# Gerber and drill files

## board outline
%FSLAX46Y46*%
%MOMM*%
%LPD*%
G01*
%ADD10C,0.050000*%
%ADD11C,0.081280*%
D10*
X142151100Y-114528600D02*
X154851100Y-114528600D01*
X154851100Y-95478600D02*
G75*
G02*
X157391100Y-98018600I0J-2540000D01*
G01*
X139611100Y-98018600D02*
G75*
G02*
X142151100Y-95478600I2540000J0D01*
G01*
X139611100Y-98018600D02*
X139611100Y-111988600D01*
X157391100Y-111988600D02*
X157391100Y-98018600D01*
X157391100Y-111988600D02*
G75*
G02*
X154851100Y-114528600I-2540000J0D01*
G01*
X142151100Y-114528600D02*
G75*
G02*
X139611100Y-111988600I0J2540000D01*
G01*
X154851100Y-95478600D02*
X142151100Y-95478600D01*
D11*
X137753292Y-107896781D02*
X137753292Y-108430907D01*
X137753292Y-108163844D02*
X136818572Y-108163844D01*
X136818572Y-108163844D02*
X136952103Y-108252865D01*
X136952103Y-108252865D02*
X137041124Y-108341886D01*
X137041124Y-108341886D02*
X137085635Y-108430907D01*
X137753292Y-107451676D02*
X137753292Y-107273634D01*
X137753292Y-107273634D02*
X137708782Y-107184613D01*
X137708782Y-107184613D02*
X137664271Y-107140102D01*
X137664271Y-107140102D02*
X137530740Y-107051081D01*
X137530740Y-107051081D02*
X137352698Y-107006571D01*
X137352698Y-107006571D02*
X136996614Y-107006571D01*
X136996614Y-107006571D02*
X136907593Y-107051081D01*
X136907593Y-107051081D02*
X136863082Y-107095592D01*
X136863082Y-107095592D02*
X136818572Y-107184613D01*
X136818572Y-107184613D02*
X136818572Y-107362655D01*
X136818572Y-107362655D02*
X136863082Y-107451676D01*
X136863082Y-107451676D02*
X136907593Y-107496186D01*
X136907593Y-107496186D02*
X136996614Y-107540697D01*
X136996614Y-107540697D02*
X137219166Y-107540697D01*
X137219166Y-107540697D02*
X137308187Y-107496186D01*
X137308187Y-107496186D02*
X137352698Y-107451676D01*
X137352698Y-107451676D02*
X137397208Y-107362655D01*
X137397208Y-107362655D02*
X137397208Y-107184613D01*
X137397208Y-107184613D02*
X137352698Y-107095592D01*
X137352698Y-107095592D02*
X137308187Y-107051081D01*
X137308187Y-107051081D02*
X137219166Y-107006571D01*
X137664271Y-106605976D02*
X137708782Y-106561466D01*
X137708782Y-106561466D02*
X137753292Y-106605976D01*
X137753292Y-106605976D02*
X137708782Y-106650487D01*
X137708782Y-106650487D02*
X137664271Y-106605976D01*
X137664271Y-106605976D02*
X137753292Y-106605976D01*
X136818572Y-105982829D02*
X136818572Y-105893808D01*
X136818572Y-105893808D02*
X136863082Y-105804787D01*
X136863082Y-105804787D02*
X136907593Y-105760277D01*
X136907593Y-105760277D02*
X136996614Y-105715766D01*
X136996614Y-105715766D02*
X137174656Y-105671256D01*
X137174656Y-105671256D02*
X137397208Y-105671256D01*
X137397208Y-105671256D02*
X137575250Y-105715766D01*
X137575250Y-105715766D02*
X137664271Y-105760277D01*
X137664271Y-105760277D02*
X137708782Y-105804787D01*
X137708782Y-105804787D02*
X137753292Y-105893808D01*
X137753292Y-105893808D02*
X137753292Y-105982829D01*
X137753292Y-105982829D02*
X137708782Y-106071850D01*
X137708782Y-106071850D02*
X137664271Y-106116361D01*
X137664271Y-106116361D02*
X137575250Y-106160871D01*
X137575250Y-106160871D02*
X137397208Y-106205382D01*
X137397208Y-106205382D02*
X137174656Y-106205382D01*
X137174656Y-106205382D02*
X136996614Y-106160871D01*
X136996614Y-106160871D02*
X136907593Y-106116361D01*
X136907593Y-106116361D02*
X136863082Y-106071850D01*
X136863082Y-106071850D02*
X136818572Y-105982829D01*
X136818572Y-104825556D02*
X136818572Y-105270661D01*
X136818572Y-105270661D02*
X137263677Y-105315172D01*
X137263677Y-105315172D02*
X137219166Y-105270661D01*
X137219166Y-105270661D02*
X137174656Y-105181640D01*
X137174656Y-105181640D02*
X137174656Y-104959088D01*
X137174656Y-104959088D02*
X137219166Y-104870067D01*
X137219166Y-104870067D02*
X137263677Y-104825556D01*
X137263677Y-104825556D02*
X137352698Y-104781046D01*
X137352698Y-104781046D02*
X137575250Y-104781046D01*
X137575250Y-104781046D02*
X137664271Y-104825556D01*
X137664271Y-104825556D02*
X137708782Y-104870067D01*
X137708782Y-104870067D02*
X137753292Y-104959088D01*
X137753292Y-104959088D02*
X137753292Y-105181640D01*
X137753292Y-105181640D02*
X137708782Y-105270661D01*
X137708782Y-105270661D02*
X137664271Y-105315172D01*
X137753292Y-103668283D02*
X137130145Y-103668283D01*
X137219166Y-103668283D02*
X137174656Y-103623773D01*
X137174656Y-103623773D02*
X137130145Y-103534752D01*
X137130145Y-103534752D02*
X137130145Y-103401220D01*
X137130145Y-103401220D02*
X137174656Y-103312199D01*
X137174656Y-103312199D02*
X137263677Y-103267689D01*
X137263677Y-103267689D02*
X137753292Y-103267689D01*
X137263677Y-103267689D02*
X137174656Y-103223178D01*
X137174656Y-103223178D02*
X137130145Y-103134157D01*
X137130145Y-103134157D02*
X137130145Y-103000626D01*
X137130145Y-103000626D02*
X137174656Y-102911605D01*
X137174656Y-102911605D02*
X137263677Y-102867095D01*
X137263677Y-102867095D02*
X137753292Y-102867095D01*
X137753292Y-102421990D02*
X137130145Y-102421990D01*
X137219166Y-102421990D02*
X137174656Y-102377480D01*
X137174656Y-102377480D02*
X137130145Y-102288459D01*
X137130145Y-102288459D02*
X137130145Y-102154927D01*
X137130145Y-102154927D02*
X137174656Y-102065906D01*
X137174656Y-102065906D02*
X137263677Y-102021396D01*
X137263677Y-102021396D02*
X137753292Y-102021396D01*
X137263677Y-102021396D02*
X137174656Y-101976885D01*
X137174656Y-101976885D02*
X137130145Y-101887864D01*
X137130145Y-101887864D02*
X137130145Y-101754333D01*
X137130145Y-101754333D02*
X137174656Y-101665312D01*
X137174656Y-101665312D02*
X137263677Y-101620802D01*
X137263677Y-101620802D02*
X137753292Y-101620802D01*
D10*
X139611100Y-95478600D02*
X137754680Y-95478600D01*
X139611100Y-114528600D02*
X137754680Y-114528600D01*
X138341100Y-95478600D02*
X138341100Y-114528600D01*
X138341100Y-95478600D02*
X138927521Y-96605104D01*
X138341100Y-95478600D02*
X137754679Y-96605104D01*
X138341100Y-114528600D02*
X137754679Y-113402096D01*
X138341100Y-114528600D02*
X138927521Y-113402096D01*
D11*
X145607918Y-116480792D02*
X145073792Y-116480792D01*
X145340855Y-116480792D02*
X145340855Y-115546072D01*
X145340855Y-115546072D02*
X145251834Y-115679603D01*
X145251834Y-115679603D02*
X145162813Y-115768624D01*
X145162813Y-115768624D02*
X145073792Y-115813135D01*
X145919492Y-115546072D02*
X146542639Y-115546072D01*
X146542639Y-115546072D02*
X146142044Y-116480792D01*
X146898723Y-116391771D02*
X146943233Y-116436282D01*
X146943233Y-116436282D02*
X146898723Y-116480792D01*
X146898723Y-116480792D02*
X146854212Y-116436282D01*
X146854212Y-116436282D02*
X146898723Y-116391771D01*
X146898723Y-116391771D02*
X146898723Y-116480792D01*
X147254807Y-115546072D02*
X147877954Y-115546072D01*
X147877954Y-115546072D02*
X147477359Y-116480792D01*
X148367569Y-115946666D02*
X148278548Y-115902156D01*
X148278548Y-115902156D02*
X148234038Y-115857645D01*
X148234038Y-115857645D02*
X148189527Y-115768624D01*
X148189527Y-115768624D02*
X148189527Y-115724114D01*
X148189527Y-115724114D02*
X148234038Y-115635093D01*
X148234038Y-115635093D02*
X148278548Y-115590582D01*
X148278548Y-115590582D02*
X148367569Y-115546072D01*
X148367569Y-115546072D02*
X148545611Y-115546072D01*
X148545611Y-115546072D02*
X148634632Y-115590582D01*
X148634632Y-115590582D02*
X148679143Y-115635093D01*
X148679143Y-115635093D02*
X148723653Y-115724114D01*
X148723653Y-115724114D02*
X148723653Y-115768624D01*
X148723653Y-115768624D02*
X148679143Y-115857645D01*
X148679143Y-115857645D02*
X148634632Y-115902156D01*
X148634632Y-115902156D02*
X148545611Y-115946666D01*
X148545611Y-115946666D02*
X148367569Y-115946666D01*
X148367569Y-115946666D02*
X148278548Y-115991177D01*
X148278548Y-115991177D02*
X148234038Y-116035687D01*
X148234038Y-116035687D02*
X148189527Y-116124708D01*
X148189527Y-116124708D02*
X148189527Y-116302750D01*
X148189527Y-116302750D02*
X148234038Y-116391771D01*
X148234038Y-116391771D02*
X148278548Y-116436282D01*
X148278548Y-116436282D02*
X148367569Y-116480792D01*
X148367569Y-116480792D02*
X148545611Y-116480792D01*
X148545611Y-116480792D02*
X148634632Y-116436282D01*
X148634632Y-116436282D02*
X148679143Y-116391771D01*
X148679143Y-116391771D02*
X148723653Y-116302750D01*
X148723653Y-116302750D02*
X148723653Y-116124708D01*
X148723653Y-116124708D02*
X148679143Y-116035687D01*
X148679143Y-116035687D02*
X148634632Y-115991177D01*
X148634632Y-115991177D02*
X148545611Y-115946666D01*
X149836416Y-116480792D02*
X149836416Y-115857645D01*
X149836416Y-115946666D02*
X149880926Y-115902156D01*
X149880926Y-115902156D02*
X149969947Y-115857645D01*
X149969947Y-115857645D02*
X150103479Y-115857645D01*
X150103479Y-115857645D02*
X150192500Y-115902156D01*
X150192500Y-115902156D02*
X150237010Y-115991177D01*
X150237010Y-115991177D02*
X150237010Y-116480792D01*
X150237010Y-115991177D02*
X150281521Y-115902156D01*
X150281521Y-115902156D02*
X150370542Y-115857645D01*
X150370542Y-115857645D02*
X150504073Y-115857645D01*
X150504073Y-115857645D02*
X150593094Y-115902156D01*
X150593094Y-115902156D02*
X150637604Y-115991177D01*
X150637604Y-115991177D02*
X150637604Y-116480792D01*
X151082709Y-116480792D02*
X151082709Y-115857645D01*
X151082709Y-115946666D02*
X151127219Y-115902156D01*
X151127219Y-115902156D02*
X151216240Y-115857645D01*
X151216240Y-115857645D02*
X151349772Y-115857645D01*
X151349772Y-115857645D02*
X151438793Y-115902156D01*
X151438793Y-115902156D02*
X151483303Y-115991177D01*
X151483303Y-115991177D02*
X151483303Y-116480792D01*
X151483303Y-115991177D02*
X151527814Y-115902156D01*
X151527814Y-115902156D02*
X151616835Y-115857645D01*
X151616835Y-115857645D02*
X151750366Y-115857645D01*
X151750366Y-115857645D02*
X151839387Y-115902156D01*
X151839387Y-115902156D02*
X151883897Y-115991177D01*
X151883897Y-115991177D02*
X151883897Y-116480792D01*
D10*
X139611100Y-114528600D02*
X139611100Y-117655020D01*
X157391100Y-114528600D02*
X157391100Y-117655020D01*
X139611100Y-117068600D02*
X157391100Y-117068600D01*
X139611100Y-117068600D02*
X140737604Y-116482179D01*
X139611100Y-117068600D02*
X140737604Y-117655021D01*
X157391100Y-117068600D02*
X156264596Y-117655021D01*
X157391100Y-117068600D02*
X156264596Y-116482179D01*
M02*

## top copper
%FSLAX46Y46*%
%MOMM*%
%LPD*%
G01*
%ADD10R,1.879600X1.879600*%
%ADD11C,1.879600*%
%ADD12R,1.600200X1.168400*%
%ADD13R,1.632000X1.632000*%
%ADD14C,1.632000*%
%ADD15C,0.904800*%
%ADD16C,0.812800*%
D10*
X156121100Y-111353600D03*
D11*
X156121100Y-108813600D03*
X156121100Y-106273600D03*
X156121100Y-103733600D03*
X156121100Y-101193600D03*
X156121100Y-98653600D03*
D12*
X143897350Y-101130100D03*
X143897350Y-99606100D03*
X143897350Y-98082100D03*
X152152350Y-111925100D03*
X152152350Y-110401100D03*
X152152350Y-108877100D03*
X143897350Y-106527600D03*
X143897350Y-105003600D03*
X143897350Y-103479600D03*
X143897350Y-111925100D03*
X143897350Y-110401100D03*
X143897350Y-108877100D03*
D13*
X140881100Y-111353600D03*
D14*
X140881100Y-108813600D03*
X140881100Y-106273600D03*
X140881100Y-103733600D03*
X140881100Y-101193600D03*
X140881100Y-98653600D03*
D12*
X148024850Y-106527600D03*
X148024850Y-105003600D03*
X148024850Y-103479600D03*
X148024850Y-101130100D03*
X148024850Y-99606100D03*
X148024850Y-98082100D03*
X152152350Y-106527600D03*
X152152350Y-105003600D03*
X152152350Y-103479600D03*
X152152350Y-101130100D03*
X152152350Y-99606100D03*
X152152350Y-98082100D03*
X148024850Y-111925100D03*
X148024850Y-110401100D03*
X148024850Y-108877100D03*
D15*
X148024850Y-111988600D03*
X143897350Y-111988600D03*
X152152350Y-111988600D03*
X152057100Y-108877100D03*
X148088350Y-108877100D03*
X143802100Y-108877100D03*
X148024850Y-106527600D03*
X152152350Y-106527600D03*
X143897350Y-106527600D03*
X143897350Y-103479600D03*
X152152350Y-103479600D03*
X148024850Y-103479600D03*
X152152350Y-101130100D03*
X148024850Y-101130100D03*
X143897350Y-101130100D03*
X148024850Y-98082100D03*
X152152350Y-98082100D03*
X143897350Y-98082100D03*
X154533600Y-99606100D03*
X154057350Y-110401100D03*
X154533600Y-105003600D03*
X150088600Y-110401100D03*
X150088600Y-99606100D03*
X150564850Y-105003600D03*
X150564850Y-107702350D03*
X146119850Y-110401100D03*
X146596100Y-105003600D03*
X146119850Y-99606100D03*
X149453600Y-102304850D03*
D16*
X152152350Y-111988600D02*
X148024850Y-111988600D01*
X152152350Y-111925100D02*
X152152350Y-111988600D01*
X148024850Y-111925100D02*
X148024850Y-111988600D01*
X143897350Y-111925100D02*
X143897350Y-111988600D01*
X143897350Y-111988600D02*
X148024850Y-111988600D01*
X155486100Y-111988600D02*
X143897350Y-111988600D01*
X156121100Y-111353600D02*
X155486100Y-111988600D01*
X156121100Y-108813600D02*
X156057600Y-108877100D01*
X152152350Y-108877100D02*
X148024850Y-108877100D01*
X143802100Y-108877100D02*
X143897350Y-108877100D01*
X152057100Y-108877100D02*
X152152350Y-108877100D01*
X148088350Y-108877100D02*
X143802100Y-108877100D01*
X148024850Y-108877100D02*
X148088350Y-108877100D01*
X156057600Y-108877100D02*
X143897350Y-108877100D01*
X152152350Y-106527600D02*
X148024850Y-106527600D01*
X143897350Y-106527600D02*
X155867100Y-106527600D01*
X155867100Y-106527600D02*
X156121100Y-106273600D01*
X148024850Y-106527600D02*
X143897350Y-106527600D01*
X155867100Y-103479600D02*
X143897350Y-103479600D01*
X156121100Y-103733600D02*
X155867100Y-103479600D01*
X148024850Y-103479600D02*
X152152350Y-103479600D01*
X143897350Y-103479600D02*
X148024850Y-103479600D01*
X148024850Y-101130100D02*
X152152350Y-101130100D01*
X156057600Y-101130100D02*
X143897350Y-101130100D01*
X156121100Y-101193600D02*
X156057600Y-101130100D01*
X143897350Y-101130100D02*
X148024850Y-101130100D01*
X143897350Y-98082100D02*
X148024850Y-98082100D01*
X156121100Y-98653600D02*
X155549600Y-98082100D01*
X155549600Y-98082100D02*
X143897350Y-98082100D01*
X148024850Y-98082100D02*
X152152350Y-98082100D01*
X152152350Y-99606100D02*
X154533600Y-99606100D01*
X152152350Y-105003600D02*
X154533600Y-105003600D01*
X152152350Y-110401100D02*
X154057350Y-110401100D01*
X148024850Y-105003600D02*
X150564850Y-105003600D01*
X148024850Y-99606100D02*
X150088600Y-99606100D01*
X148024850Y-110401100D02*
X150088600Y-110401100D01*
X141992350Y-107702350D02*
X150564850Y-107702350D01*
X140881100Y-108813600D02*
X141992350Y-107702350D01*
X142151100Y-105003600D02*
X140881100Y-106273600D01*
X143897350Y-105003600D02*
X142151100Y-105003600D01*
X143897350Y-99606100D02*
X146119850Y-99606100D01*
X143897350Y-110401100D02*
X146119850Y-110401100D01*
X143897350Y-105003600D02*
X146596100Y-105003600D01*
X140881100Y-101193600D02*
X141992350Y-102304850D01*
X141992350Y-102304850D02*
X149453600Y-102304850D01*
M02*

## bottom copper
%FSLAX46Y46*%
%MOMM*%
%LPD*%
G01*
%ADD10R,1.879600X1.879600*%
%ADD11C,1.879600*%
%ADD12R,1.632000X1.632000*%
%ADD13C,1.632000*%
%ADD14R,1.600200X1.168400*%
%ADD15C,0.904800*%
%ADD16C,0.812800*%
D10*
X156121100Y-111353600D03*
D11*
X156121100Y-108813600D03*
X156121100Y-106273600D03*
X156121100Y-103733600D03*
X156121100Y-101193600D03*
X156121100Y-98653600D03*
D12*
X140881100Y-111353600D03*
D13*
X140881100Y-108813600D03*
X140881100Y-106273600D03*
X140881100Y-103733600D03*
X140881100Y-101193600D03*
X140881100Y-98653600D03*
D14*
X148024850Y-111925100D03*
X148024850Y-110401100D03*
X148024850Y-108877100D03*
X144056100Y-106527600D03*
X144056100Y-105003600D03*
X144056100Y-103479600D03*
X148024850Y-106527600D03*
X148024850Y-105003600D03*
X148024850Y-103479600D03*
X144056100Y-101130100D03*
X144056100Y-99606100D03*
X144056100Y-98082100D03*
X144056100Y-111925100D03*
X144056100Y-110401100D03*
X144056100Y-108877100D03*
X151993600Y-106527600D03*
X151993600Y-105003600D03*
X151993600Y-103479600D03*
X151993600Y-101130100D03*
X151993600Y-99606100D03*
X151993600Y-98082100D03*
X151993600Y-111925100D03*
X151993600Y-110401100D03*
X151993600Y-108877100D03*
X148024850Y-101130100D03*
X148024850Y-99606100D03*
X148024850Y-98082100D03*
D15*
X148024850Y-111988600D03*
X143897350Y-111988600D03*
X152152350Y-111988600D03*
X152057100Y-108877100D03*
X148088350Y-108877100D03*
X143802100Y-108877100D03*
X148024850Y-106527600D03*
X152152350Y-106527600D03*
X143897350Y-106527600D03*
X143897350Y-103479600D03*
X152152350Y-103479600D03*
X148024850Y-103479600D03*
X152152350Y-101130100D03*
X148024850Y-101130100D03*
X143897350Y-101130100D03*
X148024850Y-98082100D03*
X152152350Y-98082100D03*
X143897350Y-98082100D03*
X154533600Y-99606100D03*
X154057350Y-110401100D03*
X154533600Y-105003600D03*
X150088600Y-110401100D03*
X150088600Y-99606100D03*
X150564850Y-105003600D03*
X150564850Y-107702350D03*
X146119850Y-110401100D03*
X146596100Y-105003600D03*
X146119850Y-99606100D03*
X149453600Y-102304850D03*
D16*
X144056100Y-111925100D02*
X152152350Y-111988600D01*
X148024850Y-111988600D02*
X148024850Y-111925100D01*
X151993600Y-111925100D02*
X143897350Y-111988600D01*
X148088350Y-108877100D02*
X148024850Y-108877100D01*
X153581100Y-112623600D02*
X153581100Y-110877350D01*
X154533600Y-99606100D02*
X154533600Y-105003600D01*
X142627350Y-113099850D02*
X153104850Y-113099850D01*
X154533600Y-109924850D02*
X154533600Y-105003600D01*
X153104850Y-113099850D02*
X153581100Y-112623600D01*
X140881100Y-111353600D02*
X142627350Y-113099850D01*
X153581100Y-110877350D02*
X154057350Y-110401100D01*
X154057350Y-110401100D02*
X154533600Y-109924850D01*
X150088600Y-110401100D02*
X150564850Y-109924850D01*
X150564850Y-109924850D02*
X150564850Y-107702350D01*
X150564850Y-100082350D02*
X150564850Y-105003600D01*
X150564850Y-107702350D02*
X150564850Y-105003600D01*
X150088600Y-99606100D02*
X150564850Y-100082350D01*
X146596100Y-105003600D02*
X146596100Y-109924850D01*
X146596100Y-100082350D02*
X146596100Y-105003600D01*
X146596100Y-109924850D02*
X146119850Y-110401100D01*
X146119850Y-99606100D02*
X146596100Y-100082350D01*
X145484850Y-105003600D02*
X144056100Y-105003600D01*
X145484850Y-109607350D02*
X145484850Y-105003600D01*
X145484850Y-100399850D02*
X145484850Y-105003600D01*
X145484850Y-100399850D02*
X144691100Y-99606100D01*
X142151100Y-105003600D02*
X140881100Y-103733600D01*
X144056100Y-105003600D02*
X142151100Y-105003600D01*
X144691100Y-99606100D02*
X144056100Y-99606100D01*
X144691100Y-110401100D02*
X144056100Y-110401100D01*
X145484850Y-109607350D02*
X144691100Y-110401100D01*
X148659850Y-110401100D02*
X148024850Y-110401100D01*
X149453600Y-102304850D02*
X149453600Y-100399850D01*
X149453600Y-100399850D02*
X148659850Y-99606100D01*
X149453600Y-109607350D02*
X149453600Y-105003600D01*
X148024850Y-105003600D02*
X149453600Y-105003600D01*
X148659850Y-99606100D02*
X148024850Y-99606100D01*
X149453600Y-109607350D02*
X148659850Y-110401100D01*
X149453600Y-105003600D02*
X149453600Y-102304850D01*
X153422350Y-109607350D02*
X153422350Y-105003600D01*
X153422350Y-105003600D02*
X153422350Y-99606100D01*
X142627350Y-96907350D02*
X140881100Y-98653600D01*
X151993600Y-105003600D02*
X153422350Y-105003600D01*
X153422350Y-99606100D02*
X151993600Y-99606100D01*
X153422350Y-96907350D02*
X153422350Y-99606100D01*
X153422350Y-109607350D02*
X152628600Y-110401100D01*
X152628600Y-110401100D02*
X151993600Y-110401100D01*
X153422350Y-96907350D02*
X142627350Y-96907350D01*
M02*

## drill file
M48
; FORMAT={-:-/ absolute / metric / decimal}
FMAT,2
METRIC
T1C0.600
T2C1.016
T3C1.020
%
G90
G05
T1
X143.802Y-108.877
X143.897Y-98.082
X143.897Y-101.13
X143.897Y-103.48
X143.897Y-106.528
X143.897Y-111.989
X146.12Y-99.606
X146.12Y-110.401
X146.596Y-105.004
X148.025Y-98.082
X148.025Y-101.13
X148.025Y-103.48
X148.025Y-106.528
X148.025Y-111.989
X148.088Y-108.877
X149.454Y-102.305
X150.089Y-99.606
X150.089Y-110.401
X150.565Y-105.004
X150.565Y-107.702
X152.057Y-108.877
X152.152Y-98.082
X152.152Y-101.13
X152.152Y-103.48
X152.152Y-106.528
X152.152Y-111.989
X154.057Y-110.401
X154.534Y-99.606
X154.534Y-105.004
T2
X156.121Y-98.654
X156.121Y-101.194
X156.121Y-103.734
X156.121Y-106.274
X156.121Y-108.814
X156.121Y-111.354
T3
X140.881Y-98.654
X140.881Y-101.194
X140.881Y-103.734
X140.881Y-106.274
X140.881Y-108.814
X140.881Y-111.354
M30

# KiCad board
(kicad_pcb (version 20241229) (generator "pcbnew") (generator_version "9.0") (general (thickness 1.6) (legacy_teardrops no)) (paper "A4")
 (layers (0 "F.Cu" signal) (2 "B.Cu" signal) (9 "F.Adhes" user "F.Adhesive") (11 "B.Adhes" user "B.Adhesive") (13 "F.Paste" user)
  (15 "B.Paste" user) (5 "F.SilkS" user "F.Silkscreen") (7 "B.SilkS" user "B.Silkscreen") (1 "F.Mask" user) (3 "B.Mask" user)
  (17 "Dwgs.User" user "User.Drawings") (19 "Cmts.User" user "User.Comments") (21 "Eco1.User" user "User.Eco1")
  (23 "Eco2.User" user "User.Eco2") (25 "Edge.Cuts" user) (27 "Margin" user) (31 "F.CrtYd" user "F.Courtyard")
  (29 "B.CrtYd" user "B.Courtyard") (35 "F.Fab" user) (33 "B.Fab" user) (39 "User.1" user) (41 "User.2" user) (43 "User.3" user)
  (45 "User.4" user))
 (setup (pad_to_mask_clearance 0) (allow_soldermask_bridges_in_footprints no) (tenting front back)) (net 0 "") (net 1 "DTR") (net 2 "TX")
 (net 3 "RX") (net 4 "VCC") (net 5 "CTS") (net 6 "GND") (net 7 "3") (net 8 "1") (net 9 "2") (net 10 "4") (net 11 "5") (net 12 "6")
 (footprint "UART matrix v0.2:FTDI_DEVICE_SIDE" (layer "F.Cu") (at 156.1211 105.0036 90)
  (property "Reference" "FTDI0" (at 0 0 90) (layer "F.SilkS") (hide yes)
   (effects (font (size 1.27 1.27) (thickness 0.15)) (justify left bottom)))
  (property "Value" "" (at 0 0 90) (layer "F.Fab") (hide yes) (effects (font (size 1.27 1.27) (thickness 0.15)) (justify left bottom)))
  (pad "P$1" thru_hole rect (at -6.35 0 90) (size 1.8796 1.8796) (drill 1.016) (layers "*.Cu" "*.Mask") (remove_unused_layers no)
   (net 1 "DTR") (solder_mask_margin 0.0508) (thermal_bridge_angle 0))
  (pad "P$2" thru_hole circle (at -3.81 0 90) (size 1.8796 1.8796) (drill 1.016) (layers "*.Cu" "*.Mask") (remove_unused_layers no)
   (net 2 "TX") (solder_mask_margin 0.0508) (thermal_bridge_angle 0))
  (pad "P$3" thru_hole circle (at -1.27 0 90) (size 1.8796 1.8796) (drill 1.016) (layers "*.Cu" "*.Mask") (remove_unused_layers no)
   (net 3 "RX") (solder_mask_margin 0.0508) (thermal_bridge_angle 0))
  (pad "P$4" thru_hole circle (at 1.27 0 90) (size 1.8796 1.8796) (drill 1.016) (layers "*.Cu" "*.Mask") (remove_unused_layers no)
   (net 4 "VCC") (solder_mask_margin 0.0508) (thermal_bridge_angle 0))
  (pad "P$5" thru_hole circle (at 3.81 0 90) (size 1.8796 1.8796) (drill 1.016) (layers "*.Cu" "*.Mask") (remove_unused_layers no)
   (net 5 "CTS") (solder_mask_margin 0.0508) (thermal_bridge_angle 0))
  (pad "P$6" thru_hole circle (at 6.35 0 90) (size 1.8796 1.8796) (drill 1.016) (layers "*.Cu" "*.Mask") (remove_unused_layers no)
   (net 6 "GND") (solder_mask_margin 0.0508) (thermal_bridge_angle 0)))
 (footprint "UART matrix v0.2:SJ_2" (layer "F.Cu") (at 143.89735 99.6061 90)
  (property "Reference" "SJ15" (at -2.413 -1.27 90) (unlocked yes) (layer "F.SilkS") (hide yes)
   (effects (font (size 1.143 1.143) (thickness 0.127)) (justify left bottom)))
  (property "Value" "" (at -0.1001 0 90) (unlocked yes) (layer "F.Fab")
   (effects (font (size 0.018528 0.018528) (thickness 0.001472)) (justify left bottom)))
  (pad "1" smd rect (at -1.524 0 90) (size 1.1684 1.6002) (layers "F.Cu" "F.Mask" "F.Paste") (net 5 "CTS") (solder_mask_margin 0.0508)
   (solder_paste_margin 0) (thermal_bridge_angle 0))
  (pad "2" smd rect (at 0 0 90) (size 1.1684 1.6002) (layers "F.Cu" "F.Mask" "F.Paste") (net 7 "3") (solder_mask_margin 0.0508)
   (solder_paste_margin 0) (thermal_bridge_angle 0))
  (pad "3" smd rect (at 1.524 0 90) (size 1.1684 1.6002) (layers "F.Cu" "F.Mask" "F.Paste") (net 6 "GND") (solder_mask_margin 0.0508)
   (solder_paste_margin 0) (thermal_bridge_angle 0)))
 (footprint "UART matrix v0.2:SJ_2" (layer "F.Cu") (at 152.15235 110.4011 90)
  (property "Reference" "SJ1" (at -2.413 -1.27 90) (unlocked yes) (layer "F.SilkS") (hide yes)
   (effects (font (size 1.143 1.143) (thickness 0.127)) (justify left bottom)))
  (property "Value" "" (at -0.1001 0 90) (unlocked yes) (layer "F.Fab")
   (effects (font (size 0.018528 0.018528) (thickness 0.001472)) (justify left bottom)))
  (pad "1" smd rect (at -1.524 0 90) (size 1.1684 1.6002) (layers "F.Cu" "F.Mask" "F.Paste") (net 1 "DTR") (solder_mask_margin 0.0508)
   (solder_paste_margin 0) (thermal_bridge_angle 0))
  (pad "2" smd rect (at 0 0 90) (size 1.1684 1.6002) (layers "F.Cu" "F.Mask" "F.Paste") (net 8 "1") (solder_mask_margin 0.0508)
   (solder_paste_margin 0) (thermal_bridge_angle 0))
  (pad "3" smd rect (at 1.524 0 90) (size 1.1684 1.6002) (layers "F.Cu" "F.Mask" "F.Paste") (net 2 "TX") (solder_mask_margin 0.0508)
   (solder_paste_margin 0) (thermal_bridge_angle 0)))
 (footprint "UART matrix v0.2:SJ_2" (layer "F.Cu") (at 143.89735 105.0036 90)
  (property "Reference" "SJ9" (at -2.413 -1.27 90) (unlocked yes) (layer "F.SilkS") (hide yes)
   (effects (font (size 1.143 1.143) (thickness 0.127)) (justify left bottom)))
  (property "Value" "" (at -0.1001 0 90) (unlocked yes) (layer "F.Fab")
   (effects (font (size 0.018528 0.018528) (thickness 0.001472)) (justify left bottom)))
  (pad "1" smd rect (at -1.524 0 90) (size 1.1684 1.6002) (layers "F.Cu" "F.Mask" "F.Paste") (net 3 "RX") (solder_mask_margin 0.0508)
   (solder_paste_margin 0) (thermal_bridge_angle 0))
  (pad "2" smd rect (at 0 0 90) (size 1.1684 1.6002) (layers "F.Cu" "F.Mask" "F.Paste") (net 7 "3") (solder_mask_margin 0.0508)
   (solder_paste_margin 0) (thermal_bridge_angle 0))
  (pad "3" smd rect (at 1.524 0 90) (size 1.1684 1.6002) (layers "F.Cu" "F.Mask" "F.Paste") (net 4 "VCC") (solder_mask_margin 0.0508)
   (solder_paste_margin 0) (thermal_bridge_angle 0)))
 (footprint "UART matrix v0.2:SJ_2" (layer "F.Cu") (at 143.89735 110.4011 90)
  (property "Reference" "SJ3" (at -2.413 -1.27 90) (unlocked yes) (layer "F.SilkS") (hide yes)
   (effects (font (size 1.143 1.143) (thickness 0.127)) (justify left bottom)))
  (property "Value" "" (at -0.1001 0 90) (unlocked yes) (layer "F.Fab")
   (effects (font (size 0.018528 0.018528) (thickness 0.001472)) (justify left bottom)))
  (pad "1" smd rect (at -1.524 0 90) (size 1.1684 1.6002) (layers "F.Cu" "F.Mask" "F.Paste") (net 1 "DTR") (solder_mask_margin 0.0508)
   (solder_paste_margin 0) (thermal_bridge_angle 0))
  (pad "2" smd rect (at 0 0 90) (size 1.1684 1.6002) (layers "F.Cu" "F.Mask" "F.Paste") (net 7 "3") (solder_mask_margin 0.0508)
   (solder_paste_margin 0) (thermal_bridge_angle 0))
  (pad "3" smd rect (at 1.524 0 90) (size 1.1684 1.6002) (layers "F.Cu" "F.Mask" "F.Paste") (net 2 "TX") (solder_mask_margin 0.0508)
   (solder_paste_margin 0) (thermal_bridge_angle 0)))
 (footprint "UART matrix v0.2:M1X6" (layer "F.Cu") (at 140.8811 111.3536 90)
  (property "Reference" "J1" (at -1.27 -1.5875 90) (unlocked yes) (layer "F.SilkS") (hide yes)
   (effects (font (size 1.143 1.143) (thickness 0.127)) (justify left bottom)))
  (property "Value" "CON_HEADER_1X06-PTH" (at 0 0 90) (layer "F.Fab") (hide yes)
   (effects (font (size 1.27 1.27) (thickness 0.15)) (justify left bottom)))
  (pad "1" thru_hole rect (at 0 0 90) (size 1.632 1.632) (drill 1.02) (layers "*.Cu" "*.Mask") (remove_unused_layers no) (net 8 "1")
   (solder_mask_margin 0.0508) (thermal_bridge_angle 0))
  (pad "2" thru_hole circle (at 2.54 0 90) (size 1.632 1.632) (drill 1.02) (layers "*.Cu" "*.Mask") (remove_unused_layers no) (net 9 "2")
   (solder_mask_margin 0.0508) (thermal_bridge_angle 0))
  (pad "3" thru_hole circle (at 5.08 0 90) (size 1.632 1.632) (drill 1.02) (layers "*.Cu" "*.Mask") (remove_unused_layers no) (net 7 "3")
   (solder_mask_margin 0.0508) (thermal_bridge_angle 0))
  (pad "4" thru_hole circle (at 7.62 0 90) (size 1.632 1.632) (drill 1.02) (layers "*.Cu" "*.Mask") (remove_unused_layers no) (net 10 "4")
   (solder_mask_margin 0.0508) (thermal_bridge_angle 0))
  (pad "5" thru_hole circle (at 10.16 0 90) (size 1.632 1.632) (drill 1.02) (layers "*.Cu" "*.Mask") (remove_unused_layers no) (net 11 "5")
   (solder_mask_margin 0.0508) (thermal_bridge_angle 0))
  (pad "6" thru_hole circle (at 12.7 0 90) (size 1.632 1.632) (drill 1.02) (layers "*.Cu" "*.Mask") (remove_unused_layers no) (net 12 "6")
   (solder_mask_margin 0.0508) (thermal_bridge_angle 0)))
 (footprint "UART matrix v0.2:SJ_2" (layer "F.Cu") (at 148.02485 105.0036 90)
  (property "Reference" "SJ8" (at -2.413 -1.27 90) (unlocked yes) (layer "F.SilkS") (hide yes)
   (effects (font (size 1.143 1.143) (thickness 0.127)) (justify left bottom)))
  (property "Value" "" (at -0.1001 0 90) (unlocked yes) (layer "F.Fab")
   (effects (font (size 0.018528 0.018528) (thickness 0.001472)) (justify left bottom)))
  (pad "1" smd rect (at -1.524 0 90) (size 1.1684 1.6002) (layers "F.Cu" "F.Mask" "F.Paste") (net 3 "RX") (solder_mask_margin 0.0508)
   (solder_paste_margin 0) (thermal_bridge_angle 0))
  (pad "2" smd rect (at 0 0 90) (size 1.1684 1.6002) (layers "F.Cu" "F.Mask" "F.Paste") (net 9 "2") (solder_mask_margin 0.0508)
   (solder_paste_margin 0) (thermal_bridge_angle 0))
  (pad "3" smd rect (at 1.524 0 90) (size 1.1684 1.6002) (layers "F.Cu" "F.Mask" "F.Paste") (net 4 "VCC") (solder_mask_margin 0.0508)
   (solder_paste_margin 0) (thermal_bridge_angle 0)))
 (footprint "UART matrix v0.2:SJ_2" (layer "F.Cu") (at 148.02485 99.6061 90)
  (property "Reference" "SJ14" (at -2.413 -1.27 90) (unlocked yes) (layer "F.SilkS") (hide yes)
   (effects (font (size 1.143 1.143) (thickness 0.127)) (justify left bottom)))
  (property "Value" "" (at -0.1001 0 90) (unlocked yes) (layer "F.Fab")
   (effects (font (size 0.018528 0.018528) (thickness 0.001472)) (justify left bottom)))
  (pad "1" smd rect (at -1.524 0 90) (size 1.1684 1.6002) (layers "F.Cu" "F.Mask" "F.Paste") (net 5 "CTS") (solder_mask_margin 0.0508)
   (solder_paste_margin 0) (thermal_bridge_angle 0))
  (pad "2" smd rect (at 0 0 90) (size 1.1684 1.6002) (layers "F.Cu" "F.Mask" "F.Paste") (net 9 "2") (solder_mask_margin 0.0508)
   (solder_paste_margin 0) (thermal_bridge_angle 0))
  (pad "3" smd rect (at 1.524 0 90) (size 1.1684 1.6002) (layers "F.Cu" "F.Mask" "F.Paste") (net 6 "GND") (solder_mask_margin 0.0508)
   (solder_paste_margin 0) (thermal_bridge_angle 0)))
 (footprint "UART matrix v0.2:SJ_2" (layer "F.Cu") (at 152.15235 105.0036 90)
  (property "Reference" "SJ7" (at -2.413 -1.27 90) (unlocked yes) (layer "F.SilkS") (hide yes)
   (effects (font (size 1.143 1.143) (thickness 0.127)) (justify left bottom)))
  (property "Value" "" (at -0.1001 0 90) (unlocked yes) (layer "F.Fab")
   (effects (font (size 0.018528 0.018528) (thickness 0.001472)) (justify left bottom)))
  (pad "1" smd rect (at -1.524 0 90) (size 1.1684 1.6002) (layers "F.Cu" "F.Mask" "F.Paste") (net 3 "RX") (solder_mask_margin 0.0508)
   (solder_paste_margin 0) (thermal_bridge_angle 0))
  (pad "2" smd rect (at 0 0 90) (size 1.1684 1.6002) (layers "F.Cu" "F.Mask" "F.Paste") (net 8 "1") (solder_mask_margin 0.0508)
   (solder_paste_margin 0) (thermal_bridge_angle 0))
  (pad "3" smd rect (at 1.524 0 90) (size 1.1684 1.6002) (layers "F.Cu" "F.Mask" "F.Paste") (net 4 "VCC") (solder_mask_margin 0.0508)
   (solder_paste_margin 0) (thermal_bridge_angle 0)))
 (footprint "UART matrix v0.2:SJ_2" (layer "F.Cu") (at 152.15235 99.6061 90)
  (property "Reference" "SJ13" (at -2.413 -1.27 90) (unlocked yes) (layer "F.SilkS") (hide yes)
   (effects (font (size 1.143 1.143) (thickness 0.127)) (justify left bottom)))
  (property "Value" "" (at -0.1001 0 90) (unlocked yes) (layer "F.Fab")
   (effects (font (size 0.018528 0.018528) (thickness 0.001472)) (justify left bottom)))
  (pad "1" smd rect (at -1.524 0 90) (size 1.1684 1.6002) (layers "F.Cu" "F.Mask" "F.Paste") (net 5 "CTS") (solder_mask_margin 0.0508)
   (solder_paste_margin 0) (thermal_bridge_angle 0))
  (pad "2" smd rect (at 0 0 90) (size 1.1684 1.6002) (layers "F.Cu" "F.Mask" "F.Paste") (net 8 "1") (solder_mask_margin 0.0508)
   (solder_paste_margin 0) (thermal_bridge_angle 0))
  (pad "3" smd rect (at 1.524 0 90) (size 1.1684 1.6002) (layers "F.Cu" "F.Mask" "F.Paste") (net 6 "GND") (solder_mask_margin 0.0508)
   (solder_paste_margin 0) (thermal_bridge_angle 0)))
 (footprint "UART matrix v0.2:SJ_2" (layer "F.Cu") (at 148.02485 110.4011 90)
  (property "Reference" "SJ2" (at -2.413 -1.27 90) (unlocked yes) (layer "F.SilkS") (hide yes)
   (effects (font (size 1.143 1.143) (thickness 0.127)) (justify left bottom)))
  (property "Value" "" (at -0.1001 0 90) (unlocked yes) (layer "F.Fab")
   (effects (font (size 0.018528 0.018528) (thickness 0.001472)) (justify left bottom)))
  (pad "1" smd rect (at -1.524 0 90) (size 1.1684 1.6002) (layers "F.Cu" "F.Mask" "F.Paste") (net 1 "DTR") (solder_mask_margin 0.0508)
   (solder_paste_margin 0) (thermal_bridge_angle 0))
  (pad "2" smd rect (at 0 0 90) (size 1.1684 1.6002) (layers "F.Cu" "F.Mask" "F.Paste") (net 9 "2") (solder_mask_margin 0.0508)
   (solder_paste_margin 0) (thermal_bridge_angle 0))
  (pad "3" smd rect (at 1.524 0 90) (size 1.1684 1.6002) (layers "F.Cu" "F.Mask" "F.Paste") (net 2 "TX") (solder_mask_margin 0.0508)
   (solder_paste_margin 0) (thermal_bridge_angle 0)))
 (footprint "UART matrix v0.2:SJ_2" (layer "B.Cu") (at 148.02485 110.4011 90)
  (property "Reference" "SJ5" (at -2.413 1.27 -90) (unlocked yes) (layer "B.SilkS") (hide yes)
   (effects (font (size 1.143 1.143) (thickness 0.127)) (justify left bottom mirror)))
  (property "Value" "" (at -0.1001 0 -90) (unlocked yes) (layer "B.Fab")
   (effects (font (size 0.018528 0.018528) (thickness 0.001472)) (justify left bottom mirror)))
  (pad "1" smd rect (at -1.524 0 90) (size 1.1684 1.6002) (layers "B.Cu" "B.Mask" "B.Paste") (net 1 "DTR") (solder_mask_margin 0.0508)
   (solder_paste_margin 0) (thermal_bridge_angle 0))
  (pad "2" smd rect (at 0 0 90) (size 1.1684 1.6002) (layers "B.Cu" "B.Mask" "B.Paste") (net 11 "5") (solder_mask_margin 0.0508)
   (solder_paste_margin 0) (thermal_bridge_angle 0))
  (pad "3" smd rect (at 1.524 0 90) (size 1.1684 1.6002) (layers "B.Cu" "B.Mask" "B.Paste") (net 2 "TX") (solder_mask_margin 0.0508)
   (solder_paste_margin 0) (thermal_bridge_angle 0)))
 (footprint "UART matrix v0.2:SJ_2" (layer "B.Cu") (at 144.0561 105.0036 90)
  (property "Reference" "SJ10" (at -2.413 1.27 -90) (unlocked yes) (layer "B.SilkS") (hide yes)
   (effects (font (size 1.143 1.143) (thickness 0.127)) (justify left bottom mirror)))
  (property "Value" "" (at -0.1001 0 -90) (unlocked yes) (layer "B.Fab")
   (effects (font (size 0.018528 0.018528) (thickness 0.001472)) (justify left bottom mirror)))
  (pad "1" smd rect (at -1.524 0 90) (size 1.1684 1.6002) (layers "B.Cu" "B.Mask" "B.Paste") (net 3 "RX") (solder_mask_margin 0.0508)
   (solder_paste_margin 0) (thermal_bridge_angle 0))
  (pad "2" smd rect (at 0 0 90) (size 1.1684 1.6002) (layers "B.Cu" "B.Mask" "B.Paste") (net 10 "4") (solder_mask_margin 0.0508)
   (solder_paste_margin 0) (thermal_bridge_angle 0))
  (pad "3" smd rect (at 1.524 0 90) (size 1.1684 1.6002) (layers "B.Cu" "B.Mask" "B.Paste") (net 4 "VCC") (solder_mask_margin 0.0508)
   (solder_paste_margin 0) (thermal_bridge_angle 0)))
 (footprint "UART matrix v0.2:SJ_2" (layer "B.Cu") (at 148.02485 105.0036 90)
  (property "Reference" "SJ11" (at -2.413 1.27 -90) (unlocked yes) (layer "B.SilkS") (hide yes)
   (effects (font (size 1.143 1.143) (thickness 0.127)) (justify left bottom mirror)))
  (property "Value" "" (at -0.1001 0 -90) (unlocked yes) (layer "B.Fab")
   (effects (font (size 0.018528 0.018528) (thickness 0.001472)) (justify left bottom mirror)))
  (pad "1" smd rect (at -1.524 0 90) (size 1.1684 1.6002) (layers "B.Cu" "B.Mask" "B.Paste") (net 3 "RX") (solder_mask_margin 0.0508)
   (solder_paste_margin 0) (thermal_bridge_angle 0))
  (pad "2" smd rect (at 0 0 90) (size 1.1684 1.6002) (layers "B.Cu" "B.Mask" "B.Paste") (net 11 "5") (solder_mask_margin 0.0508)
   (solder_paste_margin 0) (thermal_bridge_angle 0))
  (pad "3" smd rect (at 1.524 0 90) (size 1.1684 1.6002) (layers "B.Cu" "B.Mask" "B.Paste") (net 4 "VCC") (solder_mask_margin 0.0508)
   (solder_paste_margin 0) (thermal_bridge_angle 0)))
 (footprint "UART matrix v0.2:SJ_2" (layer "B.Cu") (at 144.0561 99.6061 90)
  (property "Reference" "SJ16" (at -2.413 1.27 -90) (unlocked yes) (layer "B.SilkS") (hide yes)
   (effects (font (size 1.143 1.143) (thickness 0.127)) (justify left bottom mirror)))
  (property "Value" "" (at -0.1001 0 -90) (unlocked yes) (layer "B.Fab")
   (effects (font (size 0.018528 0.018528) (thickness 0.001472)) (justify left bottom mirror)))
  (pad "1" smd rect (at -1.524 0 90) (size 1.1684 1.6002) (layers "B.Cu" "B.Mask" "B.Paste") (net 5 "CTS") (solder_mask_margin 0.0508)
   (solder_paste_margin 0) (thermal_bridge_angle 0))
  (pad "2" smd rect (at 0 0 90) (size 1.1684 1.6002) (layers "B.Cu" "B.Mask" "B.Paste") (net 10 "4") (solder_mask_margin 0.0508)
   (solder_paste_margin 0) (thermal_bridge_angle 0))
  (pad "3" smd rect (at 1.524 0 90) (size 1.1684 1.6002) (layers "B.Cu" "B.Mask" "B.Paste") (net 6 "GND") (solder_mask_margin 0.0508)
   (solder_paste_margin 0) (thermal_bridge_angle 0)))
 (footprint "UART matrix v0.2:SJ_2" (layer "B.Cu") (at 144.0561 110.4011 90)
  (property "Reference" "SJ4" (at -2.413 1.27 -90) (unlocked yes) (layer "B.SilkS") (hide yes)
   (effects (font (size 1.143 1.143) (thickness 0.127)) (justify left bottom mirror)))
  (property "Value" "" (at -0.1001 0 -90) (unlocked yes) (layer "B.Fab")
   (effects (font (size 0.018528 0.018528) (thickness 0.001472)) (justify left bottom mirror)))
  (pad "1" smd rect (at -1.524 0 90) (size 1.1684 1.6002) (layers "B.Cu" "B.Mask" "B.Paste") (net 1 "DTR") (solder_mask_margin 0.0508)
   (solder_paste_margin 0) (thermal_bridge_angle 0))
  (pad "2" smd rect (at 0 0 90) (size 1.1684 1.6002) (layers "B.Cu" "B.Mask" "B.Paste") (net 10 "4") (solder_mask_margin 0.0508)
   (solder_paste_margin 0) (thermal_bridge_angle 0))
  (pad "3" smd rect (at 1.524 0 90) (size 1.1684 1.6002) (layers "B.Cu" "B.Mask" "B.Paste") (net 2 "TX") (solder_mask_margin 0.0508)
   (solder_paste_margin 0) (thermal_bridge_angle 0)))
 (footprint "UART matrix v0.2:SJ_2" (layer "B.Cu") (at 151.9936 105.0036 90)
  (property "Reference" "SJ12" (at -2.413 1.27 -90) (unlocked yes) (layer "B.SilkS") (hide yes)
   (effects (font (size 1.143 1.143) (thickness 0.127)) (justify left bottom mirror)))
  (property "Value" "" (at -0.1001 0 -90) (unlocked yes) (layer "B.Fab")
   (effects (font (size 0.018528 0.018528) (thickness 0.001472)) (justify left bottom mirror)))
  (pad "1" smd rect (at -1.524 0 90) (size 1.1684 1.6002) (layers "B.Cu" "B.Mask" "B.Paste") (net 3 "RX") (solder_mask_margin 0.0508)
   (solder_paste_margin 0) (thermal_bridge_angle 0))
  (pad "2" smd rect (at 0 0 90) (size 1.1684 1.6002) (layers "B.Cu" "B.Mask" "B.Paste") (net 12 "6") (solder_mask_margin 0.0508)
   (solder_paste_margin 0) (thermal_bridge_angle 0))
  (pad "3" smd rect (at 1.524 0 90) (size 1.1684 1.6002) (layers "B.Cu" "B.Mask" "B.Paste") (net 4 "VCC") (solder_mask_margin 0.0508)
   (solder_paste_margin 0) (thermal_bridge_angle 0)))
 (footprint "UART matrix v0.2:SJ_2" (layer "B.Cu") (at 151.9936 99.6061 90)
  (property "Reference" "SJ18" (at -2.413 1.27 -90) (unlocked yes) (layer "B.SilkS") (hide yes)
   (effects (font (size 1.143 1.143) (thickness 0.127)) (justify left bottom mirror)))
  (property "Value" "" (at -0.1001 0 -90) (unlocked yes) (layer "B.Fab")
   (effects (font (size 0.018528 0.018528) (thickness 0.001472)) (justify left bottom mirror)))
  (pad "1" smd rect (at -1.524 0 90) (size 1.1684 1.6002) (layers "B.Cu" "B.Mask" "B.Paste") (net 5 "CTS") (solder_mask_margin 0.0508)
   (solder_paste_margin 0) (thermal_bridge_angle 0))
  (pad "2" smd rect (at 0 0 90) (size 1.1684 1.6002) (layers "B.Cu" "B.Mask" "B.Paste") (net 12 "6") (solder_mask_margin 0.0508)
   (solder_paste_margin 0) (thermal_bridge_angle 0))
  (pad "3" smd rect (at 1.524 0 90) (size 1.1684 1.6002) (layers "B.Cu" "B.Mask" "B.Paste") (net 6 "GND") (solder_mask_margin 0.0508)
   (solder_paste_margin 0) (thermal_bridge_angle 0)))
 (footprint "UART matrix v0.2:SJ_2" (layer "B.Cu") (at 151.9936 110.4011 90)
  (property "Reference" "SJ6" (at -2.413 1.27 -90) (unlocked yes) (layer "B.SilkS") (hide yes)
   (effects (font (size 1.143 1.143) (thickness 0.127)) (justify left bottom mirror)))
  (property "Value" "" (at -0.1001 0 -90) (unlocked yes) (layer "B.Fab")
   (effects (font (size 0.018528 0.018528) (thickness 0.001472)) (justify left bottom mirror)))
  (pad "1" smd rect (at -1.524 0 90) (size 1.1684 1.6002) (layers "B.Cu" "B.Mask" "B.Paste") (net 1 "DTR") (solder_mask_margin 0.0508)
   (solder_paste_margin 0) (thermal_bridge_angle 0))
  (pad "2" smd rect (at 0 0 90) (size 1.1684 1.6002) (layers "B.Cu" "B.Mask" "B.Paste") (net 12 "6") (solder_mask_margin 0.0508)
   (solder_paste_margin 0) (thermal_bridge_angle 0))
  (pad "3" smd rect (at 1.524 0 90) (size 1.1684 1.6002) (layers "B.Cu" "B.Mask" "B.Paste") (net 2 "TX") (solder_mask_margin 0.0508)
   (solder_paste_margin 0) (thermal_bridge_angle 0)))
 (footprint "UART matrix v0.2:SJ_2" (layer "B.Cu") (at 148.02485 99.6061 90)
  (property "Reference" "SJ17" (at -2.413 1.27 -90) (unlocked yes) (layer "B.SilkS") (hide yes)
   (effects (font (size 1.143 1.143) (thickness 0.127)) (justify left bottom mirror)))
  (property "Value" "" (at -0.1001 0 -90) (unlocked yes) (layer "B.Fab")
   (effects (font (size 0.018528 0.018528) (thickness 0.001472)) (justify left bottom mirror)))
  (pad "1" smd rect (at -1.524 0 90) (size 1.1684 1.6002) (layers "B.Cu" "B.Mask" "B.Paste") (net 5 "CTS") (solder_mask_margin 0.0508)
   (solder_paste_margin 0) (thermal_bridge_angle 0))
  (pad "2" smd rect (at 0 0 90) (size 1.1684 1.6002) (layers "B.Cu" "B.Mask" "B.Paste") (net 11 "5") (solder_mask_margin 0.0508)
   (solder_paste_margin 0) (thermal_bridge_angle 0))
  (pad "3" smd rect (at 1.524 0 90) (size 1.1684 1.6002) (layers "B.Cu" "B.Mask" "B.Paste") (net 6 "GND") (solder_mask_margin 0.0508)
   (solder_paste_margin 0) (thermal_bridge_angle 0)))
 (gr_line (start 142.1511 114.5286) (end 154.8511 114.5286) (stroke (width 0.05) (type solid)) (layer "Edge.Cuts"))
 (gr_arc (start 154.8511 95.4786) (mid 156.647151 96.222549) (end 157.3911 98.0186) (stroke (width 0.05) (type solid)) (layer "Edge.Cuts"))
 (gr_arc (start 139.6111 98.0186) (mid 140.355049 96.222549) (end 142.1511 95.4786) (stroke (width 0.05) (type solid)) (layer "Edge.Cuts"))
 (gr_line (start 139.6111 98.0186) (end 139.6111 111.9886) (stroke (width 0.05) (type solid)) (layer "Edge.Cuts"))
 (gr_line (start 157.3911 111.9886) (end 157.3911 98.0186) (stroke (width 0.05) (type solid)) (layer "Edge.Cuts"))
 (gr_arc (start 157.3911 111.9886) (mid 156.647151 113.784651) (end 154.8511 114.5286) (stroke (width 0.05) (type solid))
  (layer "Edge.Cuts"))
 (gr_arc (start 142.1511 114.5286) (mid 140.355049 113.784651) (end 139.6111 111.9886) (stroke (width 0.05) (type solid))
  (layer "Edge.Cuts"))
 (gr_line (start 154.8511 95.4786) (end 142.1511 95.4786) (stroke (width 0.05) (type solid)) (layer "Edge.Cuts"))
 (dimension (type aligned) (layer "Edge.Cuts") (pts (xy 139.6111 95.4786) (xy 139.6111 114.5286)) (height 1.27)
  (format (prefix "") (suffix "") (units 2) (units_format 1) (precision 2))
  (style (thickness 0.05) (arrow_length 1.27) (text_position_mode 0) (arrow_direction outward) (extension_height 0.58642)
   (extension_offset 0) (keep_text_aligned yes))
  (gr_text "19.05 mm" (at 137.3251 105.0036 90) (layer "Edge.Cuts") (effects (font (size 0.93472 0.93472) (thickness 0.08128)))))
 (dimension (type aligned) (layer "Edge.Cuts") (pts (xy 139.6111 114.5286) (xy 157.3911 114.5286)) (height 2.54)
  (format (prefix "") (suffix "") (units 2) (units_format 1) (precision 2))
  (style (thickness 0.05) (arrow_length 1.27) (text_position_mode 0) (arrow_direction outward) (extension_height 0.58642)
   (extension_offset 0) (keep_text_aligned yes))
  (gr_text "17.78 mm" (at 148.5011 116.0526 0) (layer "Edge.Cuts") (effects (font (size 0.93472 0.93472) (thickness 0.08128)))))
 (segment (start 152.15235 111.9886) (end 148.02485 111.9886) (width 0.8128) (layer "F.Cu") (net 1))
 (segment (start 152.15235 111.9251) (end 152.15235 111.9886) (width 0.8128) (layer "F.Cu") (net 1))
 (segment (start 148.02485 111.9251) (end 148.02485 111.9886) (width 0.8128) (layer "F.Cu") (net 1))
 (segment (start 143.89735 111.9251) (end 143.89735 111.9886) (width 0.8128) (layer "F.Cu") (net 1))
 (segment (start 143.89735 111.9886) (end 148.02485 111.9886) (width 0.8128) (layer "F.Cu") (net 1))
 (segment (start 155.4861 111.9886) (end 143.89735 111.9886) (width 0.8128) (layer "F.Cu") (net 1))
 (segment (start 156.1211 111.3536) (end 155.4861 111.9886) (width 0.8128) (layer "F.Cu") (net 1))
 (via (at 148.02485 111.9886) (size 0.9048) (drill 0.6) (layers "F.Cu" "B.Cu") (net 1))
 (via (at 143.89735 111.9886) (size 0.9048) (drill 0.6) (layers "F.Cu" "B.Cu") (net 1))
 (via (at 152.15235 111.9886) (size 0.9048) (drill 0.6) (layers "F.Cu" "B.Cu") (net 1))
 (segment (start 144.0561 111.9251) (end 152.15235 111.9886) (width 0.8128) (layer "B.Cu") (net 1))
 (segment (start 148.02485 111.9886) (end 148.02485 111.9251) (width 0.8128) (layer "B.Cu") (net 1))
 (segment (start 151.9936 111.9251) (end 143.89735 111.9886) (width 0.8128) (layer "B.Cu") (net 1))
 (segment (start 156.1211 108.8136) (end 156.0576 108.8771) (width 0.8128) (layer "F.Cu") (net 2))
 (segment (start 152.15235 108.8771) (end 148.02485 108.8771) (width 0.8128) (layer "F.Cu") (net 2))
 (segment (start 143.8021 108.8771) (end 143.89735 108.8771) (width 0.8128) (layer "F.Cu") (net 2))
 (segment (start 152.0571 108.8771) (end 152.15235 108.8771) (width 0.8128) (layer "F.Cu") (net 2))
 (segment (start 148.08835 108.8771) (end 143.8021 108.8771) (width 0.8128) (layer "F.Cu") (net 2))
 (segment (start 148.02485 108.8771) (end 148.08835 108.8771) (width 0.8128) (layer "F.Cu") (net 2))
 (segment (start 156.0576 108.8771) (end 143.89735 108.8771) (width 0.8128) (layer "F.Cu") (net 2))
 (via (at 152.0571 108.8771) (size 0.9048) (drill 0.6) (layers "F.Cu" "B.Cu") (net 2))
 (via (at 148.08835 108.8771) (size 0.9048) (drill 0.6) (layers "F.Cu" "B.Cu") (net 2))
 (via (at 143.8021 108.8771) (size 0.9048) (drill 0.6) (layers "F.Cu" "B.Cu") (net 2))
 (segment (start 148.08835 108.8771) (end 148.02485 108.8771) (width 0.8128) (layer "B.Cu") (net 2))
 (segment (start 152.15235 106.5276) (end 148.02485 106.5276) (width 0.8128) (layer "F.Cu") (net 3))
 (segment (start 143.89735 106.5276) (end 155.8671 106.5276) (width 0.8128) (layer "F.Cu") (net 3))
 (segment (start 155.8671 106.5276) (end 156.1211 106.2736) (width 0.8128) (layer "F.Cu") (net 3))
 (segment (start 148.02485 106.5276) (end 143.89735 106.5276) (width 0.8128) (layer "F.Cu") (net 3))
 (via (at 148.02485 106.5276) (size 0.9048) (drill 0.6) (layers "F.Cu" "B.Cu") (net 3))
 (via (at 152.15235 106.5276) (size 0.9048) (drill 0.6) (layers "F.Cu" "B.Cu") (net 3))
 (via (at 143.89735 106.5276) (size 0.9048) (drill 0.6) (layers "F.Cu" "B.Cu") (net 3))
 (segment (start 155.8671 103.4796) (end 143.89735 103.4796) (width 0.8128) (layer "F.Cu") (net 4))
 (segment (start 156.1211 103.7336) (end 155.8671 103.4796) (width 0.8128) (layer "F.Cu") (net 4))
 (segment (start 148.02485 103.4796) (end 152.15235 103.4796) (width 0.8128) (layer "F.Cu") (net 4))
 (segment (start 143.89735 103.4796) (end 148.02485 103.4796) (width 0.8128) (layer "F.Cu") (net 4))
 (via (at 143.89735 103.4796) (size 0.9048) (drill 0.6) (layers "F.Cu" "B.Cu") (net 4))
 (via (at 152.15235 103.4796) (size 0.9048) (drill 0.6) (layers "F.Cu" "B.Cu") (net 4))
 (via (at 148.02485 103.4796) (size 0.9048) (drill 0.6) (layers "F.Cu" "B.Cu") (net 4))
 (segment (start 148.02485 101.1301) (end 152.15235 101.1301) (width 0.8128) (layer "F.Cu") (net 5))
 (segment (start 156.0576 101.1301) (end 143.89735 101.1301) (width 0.8128) (layer "F.Cu") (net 5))
 (segment (start 156.1211 101.1936) (end 156.0576 101.1301) (width 0.8128) (layer "F.Cu") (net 5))
 (segment (start 143.89735 101.1301) (end 148.02485 101.1301) (width 0.8128) (layer "F.Cu") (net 5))
 (via (at 152.15235 101.1301) (size 0.9048) (drill 0.6) (layers "F.Cu" "B.Cu") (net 5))
 (via (at 148.02485 101.1301) (size 0.9048) (drill 0.6) (layers "F.Cu" "B.Cu") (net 5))
 (via (at 143.89735 101.1301) (size 0.9048) (drill 0.6) (layers "F.Cu" "B.Cu") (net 5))
 (segment (start 143.89735 98.0821) (end 148.02485 98.0821) (width 0.8128) (layer "F.Cu") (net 6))
 (segment (start 156.1211 98.6536) (end 155.5496 98.0821) (width 0.8128) (layer "F.Cu") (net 6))
 (segment (start 155.5496 98.0821) (end 143.89735 98.0821) (width 0.8128) (layer "F.Cu") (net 6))
 (segment (start 148.02485 98.0821) (end 152.15235 98.0821) (width 0.8128) (layer "F.Cu") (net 6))
 (via (at 148.02485 98.0821) (size 0.9048) (drill 0.6) (layers "F.Cu" "B.Cu") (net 6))
 (via (at 152.15235 98.0821) (size 0.9048) (drill 0.6) (layers "F.Cu" "B.Cu") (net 6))
 (via (at 143.89735 98.0821) (size 0.9048) (drill 0.6) (layers "F.Cu" "B.Cu") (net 6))
 (segment (start 152.15235 99.6061) (end 154.5336 99.6061) (width 0.8128) (layer "F.Cu") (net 8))
 (segment (start 152.15235 105.0036) (end 154.5336 105.0036) (width 0.8128) (layer "F.Cu") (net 8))
 (segment (start 152.15235 110.4011) (end 154.05735 110.4011) (width 0.8128) (layer "F.Cu") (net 8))
 (via (at 154.5336 99.6061) (size 0.9048) (drill 0.6) (layers "F.Cu" "B.Cu") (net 8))
 (via (at 154.05735 110.4011) (size 0.9048) (drill 0.6) (layers "F.Cu" "B.Cu") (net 8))
 (via (at 154.5336 105.0036) (size 0.9048) (drill 0.6) (layers "F.Cu" "B.Cu") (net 8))
 (segment (start 153.5811 112.6236) (end 153.5811 110.87735) (width 0.8128) (layer "B.Cu") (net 8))
 (segment (start 154.5336 99.6061) (end 154.5336 105.0036) (width 0.8128) (layer "B.Cu") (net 8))
 (segment (start 142.62735 113.09985) (end 153.10485 113.09985) (width 0.8128) (layer "B.Cu") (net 8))
 (segment (start 154.5336 109.92485) (end 154.5336 105.0036) (width 0.8128) (layer "B.Cu") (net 8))
 (segment (start 153.10485 113.09985) (end 153.5811 112.6236) (width 0.8128) (layer "B.Cu") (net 8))
 (segment (start 140.8811 111.3536) (end 142.62735 113.09985) (width 0.8128) (layer "B.Cu") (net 8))
 (segment (start 153.5811 110.87735) (end 154.05735 110.4011) (width 0.8128) (layer "B.Cu") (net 8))
 (segment (start 154.05735 110.4011) (end 154.5336 109.92485) (width 0.8128) (layer "B.Cu") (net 8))
 (segment (start 148.02485 105.0036) (end 150.56485 105.0036) (width 0.8128) (layer "F.Cu") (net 9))
 (segment (start 148.02485 99.6061) (end 150.0886 99.6061) (width 0.8128) (layer "F.Cu") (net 9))
 (segment (start 148.02485 110.4011) (end 150.0886 110.4011) (width 0.8128) (layer "F.Cu") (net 9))
 (segment (start 141.99235 107.70235) (end 150.56485 107.70235) (width 0.8128) (layer "F.Cu") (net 9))
 (segment (start 140.8811 108.8136) (end 141.99235 107.70235) (width 0.8128) (layer "F.Cu") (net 9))
 (via (at 150.0886 110.4011) (size 0.9048) (drill 0.6) (layers "F.Cu" "B.Cu") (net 9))
 (via (at 150.0886 99.6061) (size 0.9048) (drill 0.6) (layers "F.Cu" "B.Cu") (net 9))
 (via (at 150.56485 105.0036) (size 0.9048) (drill 0.6) (layers "F.Cu" "B.Cu") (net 9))
 (via (at 150.56485 107.70235) (size 0.9048) (drill 0.6) (layers "F.Cu" "B.Cu") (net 9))
 (segment (start 150.0886 110.4011) (end 150.56485 109.92485) (width 0.8128) (layer "B.Cu") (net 9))
 (segment (start 150.56485 109.92485) (end 150.56485 107.70235) (width 0.8128) (layer "B.Cu") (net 9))
 (segment (start 150.56485 100.08235) (end 150.56485 105.0036) (width 0.8128) (layer "B.Cu") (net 9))
 (segment (start 150.56485 107.70235) (end 150.56485 105.0036) (width 0.8128) (layer "B.Cu") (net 9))
 (segment (start 150.0886 99.6061) (end 150.56485 100.08235) (width 0.8128) (layer "B.Cu") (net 9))
 (segment (start 142.1511 105.0036) (end 140.8811 106.2736) (width 0.8128) (layer "F.Cu") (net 7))
 (segment (start 143.89735 105.0036) (end 142.1511 105.0036) (width 0.8128) (layer "F.Cu") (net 7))
 (segment (start 143.89735 99.6061) (end 146.11985 99.6061) (width 0.8128) (layer "F.Cu") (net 7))
 (segment (start 143.89735 110.4011) (end 146.11985 110.4011) (width 0.8128) (layer "F.Cu") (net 7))
 (segment (start 143.89735 105.0036) (end 146.5961 105.0036) (width 0.8128) (layer "F.Cu") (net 7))
 (via (at 146.11985 110.4011) (size 0.9048) (drill 0.6) (layers "F.Cu" "B.Cu") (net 7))
 (via (at 146.5961 105.0036) (size 0.9048) (drill 0.6) (layers "F.Cu" "B.Cu") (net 7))
 (via (at 146.11985 99.6061) (size 0.9048) (drill 0.6) (layers "F.Cu" "B.Cu") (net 7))
 (segment (start 146.5961 105.0036) (end 146.5961 109.92485) (width 0.8128) (layer "B.Cu") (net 7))
 (segment (start 146.5961 100.08235) (end 146.5961 105.0036) (width 0.8128) (layer "B.Cu") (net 7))
 (segment (start 146.5961 109.92485) (end 146.11985 110.4011) (width 0.8128) (layer "B.Cu") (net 7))
 (segment (start 146.11985 99.6061) (end 146.5961 100.08235) (width 0.8128) (layer "B.Cu") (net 7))
 (segment (start 145.48485 105.0036) (end 144.0561 105.0036) (width 0.8128) (layer "B.Cu") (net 10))
 (segment (start 145.48485 109.60735) (end 145.48485 105.0036) (width 0.8128) (layer "B.Cu") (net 10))
 (segment (start 145.48485 100.39985) (end 145.48485 105.0036) (width 0.8128) (layer "B.Cu") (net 10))
 (segment (start 145.48485 100.39985) (end 144.6911 99.6061) (width 0.8128) (layer "B.Cu") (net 10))
 (segment (start 142.1511 105.0036) (end 140.8811 103.7336) (width 0.8128) (layer "B.Cu") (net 10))
 (segment (start 144.0561 105.0036) (end 142.1511 105.0036) (width 0.8128) (layer "B.Cu") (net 10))
 (segment (start 144.6911 99.6061) (end 144.0561 99.6061) (width 0.8128) (layer "B.Cu") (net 10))
 (segment (start 144.6911 110.4011) (end 144.0561 110.4011) (width 0.8128) (layer "B.Cu") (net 10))
 (segment (start 145.48485 109.60735) (end 144.6911 110.4011) (width 0.8128) (layer "B.Cu") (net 10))
 (segment (start 140.8811 101.1936) (end 141.99235 102.30485) (width 0.8128) (layer "F.Cu") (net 11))
 (segment (start 141.99235 102.30485) (end 149.4536 102.30485) (width 0.8128) (layer "F.Cu") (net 11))
 (via (at 149.4536 102.30485) (size 0.9048) (drill 0.6) (layers "F.Cu" "B.Cu") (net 11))
 (segment (start 148.65985 110.4011) (end 148.02485 110.4011) (width 0.8128) (layer "B.Cu") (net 11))
 (segment (start 149.4536 102.30485) (end 149.4536 100.39985) (width 0.8128) (layer "B.Cu") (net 11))
 (segment (start 149.4536 100.39985) (end 148.65985 99.6061) (width 0.8128) (layer "B.Cu") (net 11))
 (segment (start 149.4536 109.60735) (end 149.4536 105.0036) (width 0.8128) (layer "B.Cu") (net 11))
 (segment (start 148.02485 105.0036) (end 149.4536 105.0036) (width 0.8128) (layer "B.Cu") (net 11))
 (segment (start 148.65985 99.6061) (end 148.02485 99.6061) (width 0.8128) (layer "B.Cu") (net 11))
 (segment (start 149.4536 109.60735) (end 148.65985 110.4011) (width 0.8128) (layer "B.Cu") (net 11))
 (segment (start 149.4536 105.0036) (end 149.4536 102.30485) (width 0.8128) (layer "B.Cu") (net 11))
 (segment (start 153.42235 109.60735) (end 153.42235 105.0036) (width 0.8128) (layer "B.Cu") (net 12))
 (segment (start 153.42235 105.0036) (end 153.42235 99.6061) (width 0.8128) (layer "B.Cu") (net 12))
 (segment (start 142.62735 96.90735) (end 140.8811 98.6536) (width 0.8128) (layer "B.Cu") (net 12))
 (segment (start 151.9936 105.0036) (end 153.42235 105.0036) (width 0.8128) (layer "B.Cu") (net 12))
 (segment (start 153.42235 99.6061) (end 151.9936 99.6061) (width 0.8128) (layer "B.Cu") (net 12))
 (segment (start 153.42235 96.90735) (end 153.42235 99.6061) (width 0.8128) (layer "B.Cu") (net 12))
 (segment (start 153.42235 109.60735) (end 152.6286 110.4011) (width 0.8128) (layer "B.Cu") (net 12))
 (segment (start 152.6286 110.4011) (end 151.9936 110.4011) (width 0.8128) (layer "B.Cu") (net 12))
 (segment (start 153.42235 96.90735) (end 142.62735 96.90735) (width 0.8128) (layer "B.Cu") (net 12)))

